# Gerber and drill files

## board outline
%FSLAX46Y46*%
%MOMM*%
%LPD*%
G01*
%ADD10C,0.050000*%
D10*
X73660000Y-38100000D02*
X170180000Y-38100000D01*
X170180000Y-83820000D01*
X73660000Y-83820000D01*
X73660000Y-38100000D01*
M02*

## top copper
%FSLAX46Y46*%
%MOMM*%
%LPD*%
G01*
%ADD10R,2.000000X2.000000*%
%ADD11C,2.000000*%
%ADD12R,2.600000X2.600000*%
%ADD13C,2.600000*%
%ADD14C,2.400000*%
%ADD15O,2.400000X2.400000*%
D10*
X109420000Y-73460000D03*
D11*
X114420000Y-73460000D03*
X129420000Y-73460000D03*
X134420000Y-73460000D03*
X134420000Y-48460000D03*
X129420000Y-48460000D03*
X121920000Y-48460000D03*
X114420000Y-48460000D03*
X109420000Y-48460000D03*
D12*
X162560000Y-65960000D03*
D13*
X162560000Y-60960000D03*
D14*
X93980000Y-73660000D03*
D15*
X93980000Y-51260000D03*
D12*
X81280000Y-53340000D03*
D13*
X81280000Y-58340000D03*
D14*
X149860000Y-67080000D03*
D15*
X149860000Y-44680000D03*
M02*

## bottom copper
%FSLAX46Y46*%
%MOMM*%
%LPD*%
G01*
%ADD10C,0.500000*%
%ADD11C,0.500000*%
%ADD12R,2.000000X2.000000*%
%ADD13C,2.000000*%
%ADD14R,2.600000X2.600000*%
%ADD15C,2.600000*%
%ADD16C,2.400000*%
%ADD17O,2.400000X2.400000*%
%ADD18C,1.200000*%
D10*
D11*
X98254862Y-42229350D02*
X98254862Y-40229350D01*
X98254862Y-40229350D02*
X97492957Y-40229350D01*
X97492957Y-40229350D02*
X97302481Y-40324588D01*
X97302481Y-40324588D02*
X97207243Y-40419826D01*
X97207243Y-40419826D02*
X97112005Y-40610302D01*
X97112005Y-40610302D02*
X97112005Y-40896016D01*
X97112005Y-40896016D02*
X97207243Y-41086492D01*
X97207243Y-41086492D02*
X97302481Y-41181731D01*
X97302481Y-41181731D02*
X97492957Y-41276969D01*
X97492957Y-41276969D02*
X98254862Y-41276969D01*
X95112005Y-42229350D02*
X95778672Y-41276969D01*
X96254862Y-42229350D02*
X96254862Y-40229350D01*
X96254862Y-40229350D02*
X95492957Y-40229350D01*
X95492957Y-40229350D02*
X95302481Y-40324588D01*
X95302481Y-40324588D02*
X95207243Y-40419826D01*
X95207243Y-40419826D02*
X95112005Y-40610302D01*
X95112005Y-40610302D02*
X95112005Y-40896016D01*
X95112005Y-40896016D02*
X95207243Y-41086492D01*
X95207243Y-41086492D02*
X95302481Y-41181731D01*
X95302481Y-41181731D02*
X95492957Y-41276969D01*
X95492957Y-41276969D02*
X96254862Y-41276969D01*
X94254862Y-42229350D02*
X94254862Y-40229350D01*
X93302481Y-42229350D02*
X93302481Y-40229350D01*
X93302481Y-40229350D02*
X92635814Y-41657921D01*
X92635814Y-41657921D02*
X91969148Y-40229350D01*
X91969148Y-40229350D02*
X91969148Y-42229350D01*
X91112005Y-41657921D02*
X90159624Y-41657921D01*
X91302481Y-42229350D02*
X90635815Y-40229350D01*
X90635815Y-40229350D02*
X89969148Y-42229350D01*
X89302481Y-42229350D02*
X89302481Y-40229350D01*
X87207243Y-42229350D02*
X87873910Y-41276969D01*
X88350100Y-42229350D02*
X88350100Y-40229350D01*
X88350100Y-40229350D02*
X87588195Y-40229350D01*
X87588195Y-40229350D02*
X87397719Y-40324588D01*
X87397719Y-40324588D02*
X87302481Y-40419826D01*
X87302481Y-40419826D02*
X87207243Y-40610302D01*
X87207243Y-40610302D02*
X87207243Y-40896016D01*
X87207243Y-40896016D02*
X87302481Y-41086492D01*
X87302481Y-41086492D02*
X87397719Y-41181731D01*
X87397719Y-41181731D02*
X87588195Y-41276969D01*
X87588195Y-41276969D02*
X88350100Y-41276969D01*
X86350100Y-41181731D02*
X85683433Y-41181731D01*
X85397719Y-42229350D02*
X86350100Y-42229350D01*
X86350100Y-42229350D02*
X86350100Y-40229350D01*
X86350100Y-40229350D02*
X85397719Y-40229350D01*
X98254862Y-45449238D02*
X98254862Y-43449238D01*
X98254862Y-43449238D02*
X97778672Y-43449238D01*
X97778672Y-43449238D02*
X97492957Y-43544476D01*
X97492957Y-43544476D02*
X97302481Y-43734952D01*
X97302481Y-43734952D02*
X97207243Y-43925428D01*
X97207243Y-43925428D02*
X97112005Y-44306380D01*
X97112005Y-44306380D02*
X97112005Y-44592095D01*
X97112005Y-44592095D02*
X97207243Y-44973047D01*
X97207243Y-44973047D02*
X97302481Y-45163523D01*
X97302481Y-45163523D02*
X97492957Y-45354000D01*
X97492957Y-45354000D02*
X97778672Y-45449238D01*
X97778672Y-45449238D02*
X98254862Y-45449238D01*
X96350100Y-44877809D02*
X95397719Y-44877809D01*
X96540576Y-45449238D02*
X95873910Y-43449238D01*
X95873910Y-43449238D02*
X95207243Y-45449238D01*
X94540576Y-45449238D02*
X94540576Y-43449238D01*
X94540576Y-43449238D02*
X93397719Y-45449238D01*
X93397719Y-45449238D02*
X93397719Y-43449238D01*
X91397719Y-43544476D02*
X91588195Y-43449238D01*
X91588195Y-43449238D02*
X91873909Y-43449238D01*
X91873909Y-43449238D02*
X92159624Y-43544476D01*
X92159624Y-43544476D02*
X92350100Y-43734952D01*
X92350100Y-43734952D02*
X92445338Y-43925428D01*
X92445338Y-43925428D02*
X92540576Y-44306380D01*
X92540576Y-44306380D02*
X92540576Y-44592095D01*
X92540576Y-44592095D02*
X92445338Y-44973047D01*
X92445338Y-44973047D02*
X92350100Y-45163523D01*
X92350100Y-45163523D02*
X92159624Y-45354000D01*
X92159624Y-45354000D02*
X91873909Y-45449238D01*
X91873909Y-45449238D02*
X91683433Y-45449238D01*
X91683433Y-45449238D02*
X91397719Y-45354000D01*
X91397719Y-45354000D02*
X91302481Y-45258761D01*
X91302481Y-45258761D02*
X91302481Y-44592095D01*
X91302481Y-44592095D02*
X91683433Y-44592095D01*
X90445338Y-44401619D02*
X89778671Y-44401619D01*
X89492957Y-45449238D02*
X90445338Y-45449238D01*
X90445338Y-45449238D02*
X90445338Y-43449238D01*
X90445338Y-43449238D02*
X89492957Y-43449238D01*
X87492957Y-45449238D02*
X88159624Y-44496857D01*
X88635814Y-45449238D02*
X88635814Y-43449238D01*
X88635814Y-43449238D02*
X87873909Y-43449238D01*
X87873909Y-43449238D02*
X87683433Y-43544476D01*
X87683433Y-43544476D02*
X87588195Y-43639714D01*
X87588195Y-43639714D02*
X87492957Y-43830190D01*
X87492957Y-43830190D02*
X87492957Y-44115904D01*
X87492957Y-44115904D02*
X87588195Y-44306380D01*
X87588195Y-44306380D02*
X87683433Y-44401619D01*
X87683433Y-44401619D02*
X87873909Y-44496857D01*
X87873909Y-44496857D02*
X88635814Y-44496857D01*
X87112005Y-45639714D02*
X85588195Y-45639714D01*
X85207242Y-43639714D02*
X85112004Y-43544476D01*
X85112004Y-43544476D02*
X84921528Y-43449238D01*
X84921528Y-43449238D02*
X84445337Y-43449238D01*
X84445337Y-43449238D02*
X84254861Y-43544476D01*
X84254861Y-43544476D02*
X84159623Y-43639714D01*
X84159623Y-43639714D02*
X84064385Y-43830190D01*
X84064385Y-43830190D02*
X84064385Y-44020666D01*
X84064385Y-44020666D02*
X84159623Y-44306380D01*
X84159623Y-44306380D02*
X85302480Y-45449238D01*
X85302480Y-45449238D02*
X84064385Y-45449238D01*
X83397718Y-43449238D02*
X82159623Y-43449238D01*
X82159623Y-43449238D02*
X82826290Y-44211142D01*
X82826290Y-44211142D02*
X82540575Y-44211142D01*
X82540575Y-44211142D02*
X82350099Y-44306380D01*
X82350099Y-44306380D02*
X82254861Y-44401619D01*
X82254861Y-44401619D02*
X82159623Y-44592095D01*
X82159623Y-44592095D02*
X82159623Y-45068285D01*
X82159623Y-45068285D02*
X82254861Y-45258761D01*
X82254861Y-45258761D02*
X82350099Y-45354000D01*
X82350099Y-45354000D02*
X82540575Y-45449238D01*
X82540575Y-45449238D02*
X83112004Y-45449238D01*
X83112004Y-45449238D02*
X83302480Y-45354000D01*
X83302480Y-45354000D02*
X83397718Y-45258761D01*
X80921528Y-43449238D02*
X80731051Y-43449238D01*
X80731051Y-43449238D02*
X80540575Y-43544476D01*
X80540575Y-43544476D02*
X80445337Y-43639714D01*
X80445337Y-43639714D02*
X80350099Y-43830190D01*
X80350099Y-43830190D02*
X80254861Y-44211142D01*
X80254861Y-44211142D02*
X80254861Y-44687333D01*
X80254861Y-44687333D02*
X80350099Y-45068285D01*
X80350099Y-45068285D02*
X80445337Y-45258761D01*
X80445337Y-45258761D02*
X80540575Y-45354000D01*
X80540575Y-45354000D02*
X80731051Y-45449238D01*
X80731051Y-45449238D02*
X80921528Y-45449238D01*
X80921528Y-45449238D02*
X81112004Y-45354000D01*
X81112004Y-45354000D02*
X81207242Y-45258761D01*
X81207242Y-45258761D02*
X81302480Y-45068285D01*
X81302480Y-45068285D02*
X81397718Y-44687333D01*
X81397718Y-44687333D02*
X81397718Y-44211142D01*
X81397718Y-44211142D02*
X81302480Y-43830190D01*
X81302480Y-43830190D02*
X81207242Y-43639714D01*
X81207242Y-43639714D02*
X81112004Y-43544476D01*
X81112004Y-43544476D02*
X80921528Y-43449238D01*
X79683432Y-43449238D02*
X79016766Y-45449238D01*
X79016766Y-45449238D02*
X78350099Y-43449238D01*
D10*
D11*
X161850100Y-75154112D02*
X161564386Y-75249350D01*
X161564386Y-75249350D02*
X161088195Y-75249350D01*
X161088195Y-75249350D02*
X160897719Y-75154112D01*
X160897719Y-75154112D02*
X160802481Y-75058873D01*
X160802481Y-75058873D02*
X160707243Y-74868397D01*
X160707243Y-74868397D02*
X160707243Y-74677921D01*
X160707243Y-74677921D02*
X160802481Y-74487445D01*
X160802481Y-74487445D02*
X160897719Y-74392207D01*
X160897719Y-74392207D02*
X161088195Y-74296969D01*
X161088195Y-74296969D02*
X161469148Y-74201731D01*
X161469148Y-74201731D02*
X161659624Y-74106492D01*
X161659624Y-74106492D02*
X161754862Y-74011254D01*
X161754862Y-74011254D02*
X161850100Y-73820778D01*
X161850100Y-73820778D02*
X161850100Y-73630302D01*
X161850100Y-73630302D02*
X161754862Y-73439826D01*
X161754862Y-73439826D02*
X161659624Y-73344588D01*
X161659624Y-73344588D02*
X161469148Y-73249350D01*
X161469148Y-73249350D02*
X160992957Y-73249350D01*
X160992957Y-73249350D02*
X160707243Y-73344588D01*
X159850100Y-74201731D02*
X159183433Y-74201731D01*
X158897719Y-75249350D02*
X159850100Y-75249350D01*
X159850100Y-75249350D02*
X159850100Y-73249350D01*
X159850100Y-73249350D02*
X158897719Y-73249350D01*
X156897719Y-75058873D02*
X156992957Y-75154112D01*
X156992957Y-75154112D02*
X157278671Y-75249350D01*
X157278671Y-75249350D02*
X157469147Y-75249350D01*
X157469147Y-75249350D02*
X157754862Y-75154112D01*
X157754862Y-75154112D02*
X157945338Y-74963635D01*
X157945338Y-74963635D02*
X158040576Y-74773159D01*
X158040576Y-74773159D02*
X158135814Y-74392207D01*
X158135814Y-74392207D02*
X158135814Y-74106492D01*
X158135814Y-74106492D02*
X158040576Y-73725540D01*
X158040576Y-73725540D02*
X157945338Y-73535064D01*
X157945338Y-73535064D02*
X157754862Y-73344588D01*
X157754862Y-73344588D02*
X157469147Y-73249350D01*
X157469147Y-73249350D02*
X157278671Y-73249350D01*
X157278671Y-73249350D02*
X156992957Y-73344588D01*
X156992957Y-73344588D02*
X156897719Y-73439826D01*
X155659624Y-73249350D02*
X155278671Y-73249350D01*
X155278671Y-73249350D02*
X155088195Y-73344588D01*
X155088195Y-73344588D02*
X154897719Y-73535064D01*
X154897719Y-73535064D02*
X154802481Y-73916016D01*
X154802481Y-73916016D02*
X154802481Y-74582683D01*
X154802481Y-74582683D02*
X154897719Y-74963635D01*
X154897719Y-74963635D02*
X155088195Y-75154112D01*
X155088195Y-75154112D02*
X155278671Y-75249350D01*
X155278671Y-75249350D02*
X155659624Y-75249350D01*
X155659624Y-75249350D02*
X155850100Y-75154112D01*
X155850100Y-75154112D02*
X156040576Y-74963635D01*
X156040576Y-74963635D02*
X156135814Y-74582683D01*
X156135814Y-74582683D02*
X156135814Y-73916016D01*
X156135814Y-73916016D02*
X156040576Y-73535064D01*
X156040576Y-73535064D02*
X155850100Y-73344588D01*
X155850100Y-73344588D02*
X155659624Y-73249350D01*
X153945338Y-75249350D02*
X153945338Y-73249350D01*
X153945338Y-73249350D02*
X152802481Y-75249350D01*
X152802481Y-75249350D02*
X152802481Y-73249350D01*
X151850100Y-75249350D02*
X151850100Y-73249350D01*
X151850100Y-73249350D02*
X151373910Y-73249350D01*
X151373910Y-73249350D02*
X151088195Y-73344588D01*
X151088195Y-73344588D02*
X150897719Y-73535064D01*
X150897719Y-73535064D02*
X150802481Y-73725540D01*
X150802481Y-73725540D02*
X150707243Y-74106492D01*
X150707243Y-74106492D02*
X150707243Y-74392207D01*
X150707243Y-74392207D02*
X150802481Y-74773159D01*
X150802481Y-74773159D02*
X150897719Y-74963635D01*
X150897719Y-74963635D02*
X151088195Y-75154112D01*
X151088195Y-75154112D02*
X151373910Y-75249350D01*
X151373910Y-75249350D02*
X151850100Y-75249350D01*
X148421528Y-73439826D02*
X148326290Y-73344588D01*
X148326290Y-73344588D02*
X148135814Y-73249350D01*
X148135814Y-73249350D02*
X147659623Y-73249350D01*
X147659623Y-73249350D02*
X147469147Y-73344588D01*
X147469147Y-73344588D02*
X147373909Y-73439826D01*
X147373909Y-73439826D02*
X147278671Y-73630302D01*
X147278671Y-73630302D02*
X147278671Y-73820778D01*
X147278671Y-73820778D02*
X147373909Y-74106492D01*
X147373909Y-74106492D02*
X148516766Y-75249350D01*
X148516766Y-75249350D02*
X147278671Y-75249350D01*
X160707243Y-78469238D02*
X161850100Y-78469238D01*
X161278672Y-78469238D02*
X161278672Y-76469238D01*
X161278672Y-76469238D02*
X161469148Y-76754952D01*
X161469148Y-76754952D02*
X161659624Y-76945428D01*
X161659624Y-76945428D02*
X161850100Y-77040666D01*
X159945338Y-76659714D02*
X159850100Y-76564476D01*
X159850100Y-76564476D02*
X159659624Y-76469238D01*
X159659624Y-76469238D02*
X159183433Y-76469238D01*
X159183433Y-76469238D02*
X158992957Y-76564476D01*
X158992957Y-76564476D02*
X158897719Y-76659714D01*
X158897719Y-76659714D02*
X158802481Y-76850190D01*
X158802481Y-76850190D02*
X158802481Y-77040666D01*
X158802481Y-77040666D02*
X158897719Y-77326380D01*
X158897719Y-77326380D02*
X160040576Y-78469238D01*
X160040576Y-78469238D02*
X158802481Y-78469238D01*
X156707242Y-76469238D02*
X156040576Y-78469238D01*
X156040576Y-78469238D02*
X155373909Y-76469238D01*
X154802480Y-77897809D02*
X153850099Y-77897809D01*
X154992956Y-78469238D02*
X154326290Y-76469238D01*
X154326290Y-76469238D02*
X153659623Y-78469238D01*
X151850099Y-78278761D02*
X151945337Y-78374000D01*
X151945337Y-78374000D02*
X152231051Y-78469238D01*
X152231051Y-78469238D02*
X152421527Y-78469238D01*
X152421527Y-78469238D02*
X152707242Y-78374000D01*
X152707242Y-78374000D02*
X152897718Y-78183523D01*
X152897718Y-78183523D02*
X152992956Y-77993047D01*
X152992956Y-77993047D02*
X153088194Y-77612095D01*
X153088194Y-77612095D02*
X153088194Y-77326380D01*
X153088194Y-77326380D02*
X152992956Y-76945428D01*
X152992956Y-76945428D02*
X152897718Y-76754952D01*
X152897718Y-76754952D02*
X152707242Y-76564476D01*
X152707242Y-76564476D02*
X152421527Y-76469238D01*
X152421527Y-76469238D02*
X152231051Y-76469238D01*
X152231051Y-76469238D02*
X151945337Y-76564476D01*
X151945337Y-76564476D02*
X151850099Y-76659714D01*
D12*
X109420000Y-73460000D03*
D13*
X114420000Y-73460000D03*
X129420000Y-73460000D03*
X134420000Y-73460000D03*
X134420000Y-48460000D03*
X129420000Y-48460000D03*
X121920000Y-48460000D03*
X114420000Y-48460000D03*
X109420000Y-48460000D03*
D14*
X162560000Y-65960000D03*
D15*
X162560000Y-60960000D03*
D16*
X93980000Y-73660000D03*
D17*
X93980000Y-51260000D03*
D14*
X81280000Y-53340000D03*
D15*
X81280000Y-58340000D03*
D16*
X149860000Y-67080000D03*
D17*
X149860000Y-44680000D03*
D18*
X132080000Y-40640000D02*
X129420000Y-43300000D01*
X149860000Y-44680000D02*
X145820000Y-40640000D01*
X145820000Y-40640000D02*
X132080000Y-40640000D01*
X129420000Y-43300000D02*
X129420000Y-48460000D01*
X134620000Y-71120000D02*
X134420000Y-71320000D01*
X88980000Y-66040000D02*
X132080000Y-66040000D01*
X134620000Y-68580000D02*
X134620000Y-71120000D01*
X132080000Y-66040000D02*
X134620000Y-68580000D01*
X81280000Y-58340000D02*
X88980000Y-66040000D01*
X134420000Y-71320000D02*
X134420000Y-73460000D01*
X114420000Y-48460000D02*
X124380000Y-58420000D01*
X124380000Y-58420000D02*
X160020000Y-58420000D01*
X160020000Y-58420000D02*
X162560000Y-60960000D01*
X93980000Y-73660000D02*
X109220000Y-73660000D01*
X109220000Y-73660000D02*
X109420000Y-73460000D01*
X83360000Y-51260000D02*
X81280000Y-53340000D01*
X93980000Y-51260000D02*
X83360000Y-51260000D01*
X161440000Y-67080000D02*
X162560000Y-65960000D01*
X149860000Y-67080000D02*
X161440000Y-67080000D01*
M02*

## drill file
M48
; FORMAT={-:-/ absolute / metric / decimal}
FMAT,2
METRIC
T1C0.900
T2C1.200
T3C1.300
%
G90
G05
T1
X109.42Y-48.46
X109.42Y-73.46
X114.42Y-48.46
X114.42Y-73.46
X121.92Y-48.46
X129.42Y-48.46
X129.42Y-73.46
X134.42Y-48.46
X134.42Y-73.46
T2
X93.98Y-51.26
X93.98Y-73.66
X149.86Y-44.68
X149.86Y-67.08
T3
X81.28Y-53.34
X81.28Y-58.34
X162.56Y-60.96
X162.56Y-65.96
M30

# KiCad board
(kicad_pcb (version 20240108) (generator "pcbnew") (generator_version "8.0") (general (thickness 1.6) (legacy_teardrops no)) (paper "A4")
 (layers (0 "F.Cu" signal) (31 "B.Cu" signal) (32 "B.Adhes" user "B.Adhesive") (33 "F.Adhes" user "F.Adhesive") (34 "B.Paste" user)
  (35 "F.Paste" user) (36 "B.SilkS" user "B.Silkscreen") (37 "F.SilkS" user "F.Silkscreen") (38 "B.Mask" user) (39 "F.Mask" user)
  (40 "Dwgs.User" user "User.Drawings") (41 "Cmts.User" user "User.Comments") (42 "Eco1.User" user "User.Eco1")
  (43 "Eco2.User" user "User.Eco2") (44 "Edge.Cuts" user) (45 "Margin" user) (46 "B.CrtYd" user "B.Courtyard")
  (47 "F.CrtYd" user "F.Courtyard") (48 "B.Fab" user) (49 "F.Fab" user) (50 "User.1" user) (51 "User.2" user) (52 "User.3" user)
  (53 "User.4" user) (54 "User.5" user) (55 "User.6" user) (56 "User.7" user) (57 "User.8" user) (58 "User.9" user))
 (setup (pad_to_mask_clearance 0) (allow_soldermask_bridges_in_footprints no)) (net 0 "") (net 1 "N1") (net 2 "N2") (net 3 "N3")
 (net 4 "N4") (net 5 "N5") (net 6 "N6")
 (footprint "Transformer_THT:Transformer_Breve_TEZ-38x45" (layer "F.Cu") (at 109.42 73.46)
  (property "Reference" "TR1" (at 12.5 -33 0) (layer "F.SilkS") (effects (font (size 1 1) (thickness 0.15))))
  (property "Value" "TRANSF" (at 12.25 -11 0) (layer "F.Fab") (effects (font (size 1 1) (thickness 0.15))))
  (pad "1" thru_hole rect (at 0 0) (size 2 2) (drill 0.9) (layers "*.Cu" "*.Mask") (remove_unused_layers no) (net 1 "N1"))
  (pad "2" thru_hole circle (at 5 0) (size 2 2) (drill 0.9) (layers "*.Cu" "*.Mask") (remove_unused_layers no))
  (pad "4" thru_hole circle (at 20 0) (size 2 2) (drill 0.9) (layers "*.Cu" "*.Mask") (remove_unused_layers no))
  (pad "5" thru_hole circle (at 25 0) (size 2 2) (drill 0.9) (layers "*.Cu" "*.Mask") (remove_unused_layers no) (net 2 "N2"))
  (pad "6" thru_hole circle (at 25 -25) (size 2 2) (drill 0.9) (layers "*.Cu" "*.Mask") (remove_unused_layers no))
  (pad "7" thru_hole circle (at 20 -25) (size 2 2) (drill 0.9) (layers "*.Cu" "*.Mask") (remove_unused_layers no) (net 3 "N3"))
  (pad "8" thru_hole circle (at 12.5 -25) (size 2 2) (drill 0.9) (layers "*.Cu" "*.Mask") (remove_unused_layers no))
  (pad "9" thru_hole circle (at 5 -25) (size 2 2) (drill 0.9) (layers "*.Cu" "*.Mask") (remove_unused_layers no) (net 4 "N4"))
  (pad "10" thru_hole circle (at 0 -25) (size 2 2) (drill 0.9) (layers "*.Cu" "*.Mask") (remove_unused_layers no)))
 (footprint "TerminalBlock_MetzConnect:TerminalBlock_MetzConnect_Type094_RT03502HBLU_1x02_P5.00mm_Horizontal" (layer "F.Cu")
  (at 162.56 65.96 90)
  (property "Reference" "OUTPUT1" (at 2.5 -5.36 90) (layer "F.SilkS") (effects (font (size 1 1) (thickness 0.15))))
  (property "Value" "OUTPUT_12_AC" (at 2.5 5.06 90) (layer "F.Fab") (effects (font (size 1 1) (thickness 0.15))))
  (pad "1" thru_hole rect (at 0 0 90) (size 2.6 2.6) (drill 1.3) (layers "*.Cu" "*.Mask") (remove_unused_layers no) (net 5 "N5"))
  (pad "2" thru_hole circle (at 5 0 90) (size 2.6 2.6) (drill 1.3) (layers "*.Cu" "*.Mask") (remove_unused_layers no) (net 4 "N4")))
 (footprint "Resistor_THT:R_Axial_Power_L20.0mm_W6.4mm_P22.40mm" (layer "F.Cu") (at 93.98 73.66 90)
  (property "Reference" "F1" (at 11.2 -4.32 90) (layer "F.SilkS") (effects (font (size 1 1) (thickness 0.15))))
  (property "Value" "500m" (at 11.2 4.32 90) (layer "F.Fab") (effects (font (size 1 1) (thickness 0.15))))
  (pad "1" thru_hole circle (at 0 0 90) (size 2.4 2.4) (drill 1.2) (layers "*.Cu" "*.Mask") (remove_unused_layers no) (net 1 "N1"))
  (pad "2" thru_hole oval (at 22.4 0 90) (size 2.4 2.4) (drill 1.2) (layers "*.Cu" "*.Mask") (remove_unused_layers no) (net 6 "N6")))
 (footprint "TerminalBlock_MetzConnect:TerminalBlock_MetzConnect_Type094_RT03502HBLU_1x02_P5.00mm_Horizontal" (layer "F.Cu")
  (at 81.28 53.34 -90)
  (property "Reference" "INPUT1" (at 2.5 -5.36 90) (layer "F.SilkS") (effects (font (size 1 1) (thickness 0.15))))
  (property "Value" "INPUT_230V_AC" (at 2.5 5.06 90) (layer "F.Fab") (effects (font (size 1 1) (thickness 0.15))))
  (pad "1" thru_hole rect (at 0 0 270) (size 2.6 2.6) (drill 1.3) (layers "*.Cu" "*.Mask") (remove_unused_layers no) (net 6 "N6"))
  (pad "2" thru_hole circle (at 5 0 270) (size 2.6 2.6) (drill 1.3) (layers "*.Cu" "*.Mask") (remove_unused_layers no) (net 2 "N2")))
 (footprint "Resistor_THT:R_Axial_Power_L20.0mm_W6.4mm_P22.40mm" (layer "F.Cu") (at 149.86 67.08 90)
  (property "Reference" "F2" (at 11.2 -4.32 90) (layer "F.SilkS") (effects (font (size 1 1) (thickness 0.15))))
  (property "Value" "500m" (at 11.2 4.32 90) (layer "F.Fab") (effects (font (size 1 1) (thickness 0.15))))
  (pad "1" thru_hole circle (at 0 0 90) (size 2.4 2.4) (drill 1.2) (layers "*.Cu" "*.Mask") (remove_unused_layers no) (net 5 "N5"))
  (pad "2" thru_hole oval (at 22.4 0 90) (size 2.4 2.4) (drill 1.2) (layers "*.Cu" "*.Mask") (remove_unused_layers no) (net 3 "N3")))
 (gr_rect (start 73.66 38.1) (end 170.18 83.82) (stroke (width 0.05) (type default)) (fill none) (layer "Edge.Cuts"))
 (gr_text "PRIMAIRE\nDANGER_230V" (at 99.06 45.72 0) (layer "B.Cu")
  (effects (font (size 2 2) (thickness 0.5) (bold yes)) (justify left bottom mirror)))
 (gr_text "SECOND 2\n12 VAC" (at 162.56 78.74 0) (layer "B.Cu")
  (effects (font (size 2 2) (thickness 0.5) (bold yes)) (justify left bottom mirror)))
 (segment (start 132.08 40.64) (end 129.42 43.3) (width 1.2) (layer "B.Cu") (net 3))
 (segment (start 149.86 44.68) (end 145.82 40.64) (width 1.2) (layer "B.Cu") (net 3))
 (segment (start 145.82 40.64) (end 132.08 40.64) (width 1.2) (layer "B.Cu") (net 3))
 (segment (start 129.42 43.3) (end 129.42 48.46) (width 1.2) (layer "B.Cu") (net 3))
 (segment (start 134.62 71.12) (end 134.42 71.32) (width 1.2) (layer "B.Cu") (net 2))
 (segment (start 88.98 66.04) (end 132.08 66.04) (width 1.2) (layer "B.Cu") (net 2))
 (segment (start 134.62 68.58) (end 134.62 71.12) (width 1.2) (layer "B.Cu") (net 2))
 (segment (start 132.08 66.04) (end 134.62 68.58) (width 1.2) (layer "B.Cu") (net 2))
 (segment (start 81.28 58.34) (end 88.98 66.04) (width 1.2) (layer "B.Cu") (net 2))
 (segment (start 134.42 71.32) (end 134.42 73.46) (width 1.2) (layer "B.Cu") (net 2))
 (segment (start 114.42 48.46) (end 124.38 58.42) (width 1.2) (layer "B.Cu") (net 4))
 (segment (start 124.38 58.42) (end 160.02 58.42) (width 1.2) (layer "B.Cu") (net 4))
 (segment (start 160.02 58.42) (end 162.56 60.96) (width 1.2) (layer "B.Cu") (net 4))
 (segment (start 93.98 73.66) (end 109.22 73.66) (width 1.2) (layer "B.Cu") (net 1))
 (segment (start 109.22 73.66) (end 109.42 73.46) (width 1.2) (layer "B.Cu") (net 1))
 (segment (start 83.36 51.26) (end 81.28 53.34) (width 1.2) (layer "B.Cu") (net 6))
 (segment (start 93.98 51.26) (end 83.36 51.26) (width 1.2) (layer "B.Cu") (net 6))
 (segment (start 161.44 67.08) (end 162.56 65.96) (width 1.2) (layer "B.Cu") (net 5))
 (segment (start 149.86 67.08) (end 161.44 67.08) (width 1.2) (layer "B.Cu") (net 5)))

